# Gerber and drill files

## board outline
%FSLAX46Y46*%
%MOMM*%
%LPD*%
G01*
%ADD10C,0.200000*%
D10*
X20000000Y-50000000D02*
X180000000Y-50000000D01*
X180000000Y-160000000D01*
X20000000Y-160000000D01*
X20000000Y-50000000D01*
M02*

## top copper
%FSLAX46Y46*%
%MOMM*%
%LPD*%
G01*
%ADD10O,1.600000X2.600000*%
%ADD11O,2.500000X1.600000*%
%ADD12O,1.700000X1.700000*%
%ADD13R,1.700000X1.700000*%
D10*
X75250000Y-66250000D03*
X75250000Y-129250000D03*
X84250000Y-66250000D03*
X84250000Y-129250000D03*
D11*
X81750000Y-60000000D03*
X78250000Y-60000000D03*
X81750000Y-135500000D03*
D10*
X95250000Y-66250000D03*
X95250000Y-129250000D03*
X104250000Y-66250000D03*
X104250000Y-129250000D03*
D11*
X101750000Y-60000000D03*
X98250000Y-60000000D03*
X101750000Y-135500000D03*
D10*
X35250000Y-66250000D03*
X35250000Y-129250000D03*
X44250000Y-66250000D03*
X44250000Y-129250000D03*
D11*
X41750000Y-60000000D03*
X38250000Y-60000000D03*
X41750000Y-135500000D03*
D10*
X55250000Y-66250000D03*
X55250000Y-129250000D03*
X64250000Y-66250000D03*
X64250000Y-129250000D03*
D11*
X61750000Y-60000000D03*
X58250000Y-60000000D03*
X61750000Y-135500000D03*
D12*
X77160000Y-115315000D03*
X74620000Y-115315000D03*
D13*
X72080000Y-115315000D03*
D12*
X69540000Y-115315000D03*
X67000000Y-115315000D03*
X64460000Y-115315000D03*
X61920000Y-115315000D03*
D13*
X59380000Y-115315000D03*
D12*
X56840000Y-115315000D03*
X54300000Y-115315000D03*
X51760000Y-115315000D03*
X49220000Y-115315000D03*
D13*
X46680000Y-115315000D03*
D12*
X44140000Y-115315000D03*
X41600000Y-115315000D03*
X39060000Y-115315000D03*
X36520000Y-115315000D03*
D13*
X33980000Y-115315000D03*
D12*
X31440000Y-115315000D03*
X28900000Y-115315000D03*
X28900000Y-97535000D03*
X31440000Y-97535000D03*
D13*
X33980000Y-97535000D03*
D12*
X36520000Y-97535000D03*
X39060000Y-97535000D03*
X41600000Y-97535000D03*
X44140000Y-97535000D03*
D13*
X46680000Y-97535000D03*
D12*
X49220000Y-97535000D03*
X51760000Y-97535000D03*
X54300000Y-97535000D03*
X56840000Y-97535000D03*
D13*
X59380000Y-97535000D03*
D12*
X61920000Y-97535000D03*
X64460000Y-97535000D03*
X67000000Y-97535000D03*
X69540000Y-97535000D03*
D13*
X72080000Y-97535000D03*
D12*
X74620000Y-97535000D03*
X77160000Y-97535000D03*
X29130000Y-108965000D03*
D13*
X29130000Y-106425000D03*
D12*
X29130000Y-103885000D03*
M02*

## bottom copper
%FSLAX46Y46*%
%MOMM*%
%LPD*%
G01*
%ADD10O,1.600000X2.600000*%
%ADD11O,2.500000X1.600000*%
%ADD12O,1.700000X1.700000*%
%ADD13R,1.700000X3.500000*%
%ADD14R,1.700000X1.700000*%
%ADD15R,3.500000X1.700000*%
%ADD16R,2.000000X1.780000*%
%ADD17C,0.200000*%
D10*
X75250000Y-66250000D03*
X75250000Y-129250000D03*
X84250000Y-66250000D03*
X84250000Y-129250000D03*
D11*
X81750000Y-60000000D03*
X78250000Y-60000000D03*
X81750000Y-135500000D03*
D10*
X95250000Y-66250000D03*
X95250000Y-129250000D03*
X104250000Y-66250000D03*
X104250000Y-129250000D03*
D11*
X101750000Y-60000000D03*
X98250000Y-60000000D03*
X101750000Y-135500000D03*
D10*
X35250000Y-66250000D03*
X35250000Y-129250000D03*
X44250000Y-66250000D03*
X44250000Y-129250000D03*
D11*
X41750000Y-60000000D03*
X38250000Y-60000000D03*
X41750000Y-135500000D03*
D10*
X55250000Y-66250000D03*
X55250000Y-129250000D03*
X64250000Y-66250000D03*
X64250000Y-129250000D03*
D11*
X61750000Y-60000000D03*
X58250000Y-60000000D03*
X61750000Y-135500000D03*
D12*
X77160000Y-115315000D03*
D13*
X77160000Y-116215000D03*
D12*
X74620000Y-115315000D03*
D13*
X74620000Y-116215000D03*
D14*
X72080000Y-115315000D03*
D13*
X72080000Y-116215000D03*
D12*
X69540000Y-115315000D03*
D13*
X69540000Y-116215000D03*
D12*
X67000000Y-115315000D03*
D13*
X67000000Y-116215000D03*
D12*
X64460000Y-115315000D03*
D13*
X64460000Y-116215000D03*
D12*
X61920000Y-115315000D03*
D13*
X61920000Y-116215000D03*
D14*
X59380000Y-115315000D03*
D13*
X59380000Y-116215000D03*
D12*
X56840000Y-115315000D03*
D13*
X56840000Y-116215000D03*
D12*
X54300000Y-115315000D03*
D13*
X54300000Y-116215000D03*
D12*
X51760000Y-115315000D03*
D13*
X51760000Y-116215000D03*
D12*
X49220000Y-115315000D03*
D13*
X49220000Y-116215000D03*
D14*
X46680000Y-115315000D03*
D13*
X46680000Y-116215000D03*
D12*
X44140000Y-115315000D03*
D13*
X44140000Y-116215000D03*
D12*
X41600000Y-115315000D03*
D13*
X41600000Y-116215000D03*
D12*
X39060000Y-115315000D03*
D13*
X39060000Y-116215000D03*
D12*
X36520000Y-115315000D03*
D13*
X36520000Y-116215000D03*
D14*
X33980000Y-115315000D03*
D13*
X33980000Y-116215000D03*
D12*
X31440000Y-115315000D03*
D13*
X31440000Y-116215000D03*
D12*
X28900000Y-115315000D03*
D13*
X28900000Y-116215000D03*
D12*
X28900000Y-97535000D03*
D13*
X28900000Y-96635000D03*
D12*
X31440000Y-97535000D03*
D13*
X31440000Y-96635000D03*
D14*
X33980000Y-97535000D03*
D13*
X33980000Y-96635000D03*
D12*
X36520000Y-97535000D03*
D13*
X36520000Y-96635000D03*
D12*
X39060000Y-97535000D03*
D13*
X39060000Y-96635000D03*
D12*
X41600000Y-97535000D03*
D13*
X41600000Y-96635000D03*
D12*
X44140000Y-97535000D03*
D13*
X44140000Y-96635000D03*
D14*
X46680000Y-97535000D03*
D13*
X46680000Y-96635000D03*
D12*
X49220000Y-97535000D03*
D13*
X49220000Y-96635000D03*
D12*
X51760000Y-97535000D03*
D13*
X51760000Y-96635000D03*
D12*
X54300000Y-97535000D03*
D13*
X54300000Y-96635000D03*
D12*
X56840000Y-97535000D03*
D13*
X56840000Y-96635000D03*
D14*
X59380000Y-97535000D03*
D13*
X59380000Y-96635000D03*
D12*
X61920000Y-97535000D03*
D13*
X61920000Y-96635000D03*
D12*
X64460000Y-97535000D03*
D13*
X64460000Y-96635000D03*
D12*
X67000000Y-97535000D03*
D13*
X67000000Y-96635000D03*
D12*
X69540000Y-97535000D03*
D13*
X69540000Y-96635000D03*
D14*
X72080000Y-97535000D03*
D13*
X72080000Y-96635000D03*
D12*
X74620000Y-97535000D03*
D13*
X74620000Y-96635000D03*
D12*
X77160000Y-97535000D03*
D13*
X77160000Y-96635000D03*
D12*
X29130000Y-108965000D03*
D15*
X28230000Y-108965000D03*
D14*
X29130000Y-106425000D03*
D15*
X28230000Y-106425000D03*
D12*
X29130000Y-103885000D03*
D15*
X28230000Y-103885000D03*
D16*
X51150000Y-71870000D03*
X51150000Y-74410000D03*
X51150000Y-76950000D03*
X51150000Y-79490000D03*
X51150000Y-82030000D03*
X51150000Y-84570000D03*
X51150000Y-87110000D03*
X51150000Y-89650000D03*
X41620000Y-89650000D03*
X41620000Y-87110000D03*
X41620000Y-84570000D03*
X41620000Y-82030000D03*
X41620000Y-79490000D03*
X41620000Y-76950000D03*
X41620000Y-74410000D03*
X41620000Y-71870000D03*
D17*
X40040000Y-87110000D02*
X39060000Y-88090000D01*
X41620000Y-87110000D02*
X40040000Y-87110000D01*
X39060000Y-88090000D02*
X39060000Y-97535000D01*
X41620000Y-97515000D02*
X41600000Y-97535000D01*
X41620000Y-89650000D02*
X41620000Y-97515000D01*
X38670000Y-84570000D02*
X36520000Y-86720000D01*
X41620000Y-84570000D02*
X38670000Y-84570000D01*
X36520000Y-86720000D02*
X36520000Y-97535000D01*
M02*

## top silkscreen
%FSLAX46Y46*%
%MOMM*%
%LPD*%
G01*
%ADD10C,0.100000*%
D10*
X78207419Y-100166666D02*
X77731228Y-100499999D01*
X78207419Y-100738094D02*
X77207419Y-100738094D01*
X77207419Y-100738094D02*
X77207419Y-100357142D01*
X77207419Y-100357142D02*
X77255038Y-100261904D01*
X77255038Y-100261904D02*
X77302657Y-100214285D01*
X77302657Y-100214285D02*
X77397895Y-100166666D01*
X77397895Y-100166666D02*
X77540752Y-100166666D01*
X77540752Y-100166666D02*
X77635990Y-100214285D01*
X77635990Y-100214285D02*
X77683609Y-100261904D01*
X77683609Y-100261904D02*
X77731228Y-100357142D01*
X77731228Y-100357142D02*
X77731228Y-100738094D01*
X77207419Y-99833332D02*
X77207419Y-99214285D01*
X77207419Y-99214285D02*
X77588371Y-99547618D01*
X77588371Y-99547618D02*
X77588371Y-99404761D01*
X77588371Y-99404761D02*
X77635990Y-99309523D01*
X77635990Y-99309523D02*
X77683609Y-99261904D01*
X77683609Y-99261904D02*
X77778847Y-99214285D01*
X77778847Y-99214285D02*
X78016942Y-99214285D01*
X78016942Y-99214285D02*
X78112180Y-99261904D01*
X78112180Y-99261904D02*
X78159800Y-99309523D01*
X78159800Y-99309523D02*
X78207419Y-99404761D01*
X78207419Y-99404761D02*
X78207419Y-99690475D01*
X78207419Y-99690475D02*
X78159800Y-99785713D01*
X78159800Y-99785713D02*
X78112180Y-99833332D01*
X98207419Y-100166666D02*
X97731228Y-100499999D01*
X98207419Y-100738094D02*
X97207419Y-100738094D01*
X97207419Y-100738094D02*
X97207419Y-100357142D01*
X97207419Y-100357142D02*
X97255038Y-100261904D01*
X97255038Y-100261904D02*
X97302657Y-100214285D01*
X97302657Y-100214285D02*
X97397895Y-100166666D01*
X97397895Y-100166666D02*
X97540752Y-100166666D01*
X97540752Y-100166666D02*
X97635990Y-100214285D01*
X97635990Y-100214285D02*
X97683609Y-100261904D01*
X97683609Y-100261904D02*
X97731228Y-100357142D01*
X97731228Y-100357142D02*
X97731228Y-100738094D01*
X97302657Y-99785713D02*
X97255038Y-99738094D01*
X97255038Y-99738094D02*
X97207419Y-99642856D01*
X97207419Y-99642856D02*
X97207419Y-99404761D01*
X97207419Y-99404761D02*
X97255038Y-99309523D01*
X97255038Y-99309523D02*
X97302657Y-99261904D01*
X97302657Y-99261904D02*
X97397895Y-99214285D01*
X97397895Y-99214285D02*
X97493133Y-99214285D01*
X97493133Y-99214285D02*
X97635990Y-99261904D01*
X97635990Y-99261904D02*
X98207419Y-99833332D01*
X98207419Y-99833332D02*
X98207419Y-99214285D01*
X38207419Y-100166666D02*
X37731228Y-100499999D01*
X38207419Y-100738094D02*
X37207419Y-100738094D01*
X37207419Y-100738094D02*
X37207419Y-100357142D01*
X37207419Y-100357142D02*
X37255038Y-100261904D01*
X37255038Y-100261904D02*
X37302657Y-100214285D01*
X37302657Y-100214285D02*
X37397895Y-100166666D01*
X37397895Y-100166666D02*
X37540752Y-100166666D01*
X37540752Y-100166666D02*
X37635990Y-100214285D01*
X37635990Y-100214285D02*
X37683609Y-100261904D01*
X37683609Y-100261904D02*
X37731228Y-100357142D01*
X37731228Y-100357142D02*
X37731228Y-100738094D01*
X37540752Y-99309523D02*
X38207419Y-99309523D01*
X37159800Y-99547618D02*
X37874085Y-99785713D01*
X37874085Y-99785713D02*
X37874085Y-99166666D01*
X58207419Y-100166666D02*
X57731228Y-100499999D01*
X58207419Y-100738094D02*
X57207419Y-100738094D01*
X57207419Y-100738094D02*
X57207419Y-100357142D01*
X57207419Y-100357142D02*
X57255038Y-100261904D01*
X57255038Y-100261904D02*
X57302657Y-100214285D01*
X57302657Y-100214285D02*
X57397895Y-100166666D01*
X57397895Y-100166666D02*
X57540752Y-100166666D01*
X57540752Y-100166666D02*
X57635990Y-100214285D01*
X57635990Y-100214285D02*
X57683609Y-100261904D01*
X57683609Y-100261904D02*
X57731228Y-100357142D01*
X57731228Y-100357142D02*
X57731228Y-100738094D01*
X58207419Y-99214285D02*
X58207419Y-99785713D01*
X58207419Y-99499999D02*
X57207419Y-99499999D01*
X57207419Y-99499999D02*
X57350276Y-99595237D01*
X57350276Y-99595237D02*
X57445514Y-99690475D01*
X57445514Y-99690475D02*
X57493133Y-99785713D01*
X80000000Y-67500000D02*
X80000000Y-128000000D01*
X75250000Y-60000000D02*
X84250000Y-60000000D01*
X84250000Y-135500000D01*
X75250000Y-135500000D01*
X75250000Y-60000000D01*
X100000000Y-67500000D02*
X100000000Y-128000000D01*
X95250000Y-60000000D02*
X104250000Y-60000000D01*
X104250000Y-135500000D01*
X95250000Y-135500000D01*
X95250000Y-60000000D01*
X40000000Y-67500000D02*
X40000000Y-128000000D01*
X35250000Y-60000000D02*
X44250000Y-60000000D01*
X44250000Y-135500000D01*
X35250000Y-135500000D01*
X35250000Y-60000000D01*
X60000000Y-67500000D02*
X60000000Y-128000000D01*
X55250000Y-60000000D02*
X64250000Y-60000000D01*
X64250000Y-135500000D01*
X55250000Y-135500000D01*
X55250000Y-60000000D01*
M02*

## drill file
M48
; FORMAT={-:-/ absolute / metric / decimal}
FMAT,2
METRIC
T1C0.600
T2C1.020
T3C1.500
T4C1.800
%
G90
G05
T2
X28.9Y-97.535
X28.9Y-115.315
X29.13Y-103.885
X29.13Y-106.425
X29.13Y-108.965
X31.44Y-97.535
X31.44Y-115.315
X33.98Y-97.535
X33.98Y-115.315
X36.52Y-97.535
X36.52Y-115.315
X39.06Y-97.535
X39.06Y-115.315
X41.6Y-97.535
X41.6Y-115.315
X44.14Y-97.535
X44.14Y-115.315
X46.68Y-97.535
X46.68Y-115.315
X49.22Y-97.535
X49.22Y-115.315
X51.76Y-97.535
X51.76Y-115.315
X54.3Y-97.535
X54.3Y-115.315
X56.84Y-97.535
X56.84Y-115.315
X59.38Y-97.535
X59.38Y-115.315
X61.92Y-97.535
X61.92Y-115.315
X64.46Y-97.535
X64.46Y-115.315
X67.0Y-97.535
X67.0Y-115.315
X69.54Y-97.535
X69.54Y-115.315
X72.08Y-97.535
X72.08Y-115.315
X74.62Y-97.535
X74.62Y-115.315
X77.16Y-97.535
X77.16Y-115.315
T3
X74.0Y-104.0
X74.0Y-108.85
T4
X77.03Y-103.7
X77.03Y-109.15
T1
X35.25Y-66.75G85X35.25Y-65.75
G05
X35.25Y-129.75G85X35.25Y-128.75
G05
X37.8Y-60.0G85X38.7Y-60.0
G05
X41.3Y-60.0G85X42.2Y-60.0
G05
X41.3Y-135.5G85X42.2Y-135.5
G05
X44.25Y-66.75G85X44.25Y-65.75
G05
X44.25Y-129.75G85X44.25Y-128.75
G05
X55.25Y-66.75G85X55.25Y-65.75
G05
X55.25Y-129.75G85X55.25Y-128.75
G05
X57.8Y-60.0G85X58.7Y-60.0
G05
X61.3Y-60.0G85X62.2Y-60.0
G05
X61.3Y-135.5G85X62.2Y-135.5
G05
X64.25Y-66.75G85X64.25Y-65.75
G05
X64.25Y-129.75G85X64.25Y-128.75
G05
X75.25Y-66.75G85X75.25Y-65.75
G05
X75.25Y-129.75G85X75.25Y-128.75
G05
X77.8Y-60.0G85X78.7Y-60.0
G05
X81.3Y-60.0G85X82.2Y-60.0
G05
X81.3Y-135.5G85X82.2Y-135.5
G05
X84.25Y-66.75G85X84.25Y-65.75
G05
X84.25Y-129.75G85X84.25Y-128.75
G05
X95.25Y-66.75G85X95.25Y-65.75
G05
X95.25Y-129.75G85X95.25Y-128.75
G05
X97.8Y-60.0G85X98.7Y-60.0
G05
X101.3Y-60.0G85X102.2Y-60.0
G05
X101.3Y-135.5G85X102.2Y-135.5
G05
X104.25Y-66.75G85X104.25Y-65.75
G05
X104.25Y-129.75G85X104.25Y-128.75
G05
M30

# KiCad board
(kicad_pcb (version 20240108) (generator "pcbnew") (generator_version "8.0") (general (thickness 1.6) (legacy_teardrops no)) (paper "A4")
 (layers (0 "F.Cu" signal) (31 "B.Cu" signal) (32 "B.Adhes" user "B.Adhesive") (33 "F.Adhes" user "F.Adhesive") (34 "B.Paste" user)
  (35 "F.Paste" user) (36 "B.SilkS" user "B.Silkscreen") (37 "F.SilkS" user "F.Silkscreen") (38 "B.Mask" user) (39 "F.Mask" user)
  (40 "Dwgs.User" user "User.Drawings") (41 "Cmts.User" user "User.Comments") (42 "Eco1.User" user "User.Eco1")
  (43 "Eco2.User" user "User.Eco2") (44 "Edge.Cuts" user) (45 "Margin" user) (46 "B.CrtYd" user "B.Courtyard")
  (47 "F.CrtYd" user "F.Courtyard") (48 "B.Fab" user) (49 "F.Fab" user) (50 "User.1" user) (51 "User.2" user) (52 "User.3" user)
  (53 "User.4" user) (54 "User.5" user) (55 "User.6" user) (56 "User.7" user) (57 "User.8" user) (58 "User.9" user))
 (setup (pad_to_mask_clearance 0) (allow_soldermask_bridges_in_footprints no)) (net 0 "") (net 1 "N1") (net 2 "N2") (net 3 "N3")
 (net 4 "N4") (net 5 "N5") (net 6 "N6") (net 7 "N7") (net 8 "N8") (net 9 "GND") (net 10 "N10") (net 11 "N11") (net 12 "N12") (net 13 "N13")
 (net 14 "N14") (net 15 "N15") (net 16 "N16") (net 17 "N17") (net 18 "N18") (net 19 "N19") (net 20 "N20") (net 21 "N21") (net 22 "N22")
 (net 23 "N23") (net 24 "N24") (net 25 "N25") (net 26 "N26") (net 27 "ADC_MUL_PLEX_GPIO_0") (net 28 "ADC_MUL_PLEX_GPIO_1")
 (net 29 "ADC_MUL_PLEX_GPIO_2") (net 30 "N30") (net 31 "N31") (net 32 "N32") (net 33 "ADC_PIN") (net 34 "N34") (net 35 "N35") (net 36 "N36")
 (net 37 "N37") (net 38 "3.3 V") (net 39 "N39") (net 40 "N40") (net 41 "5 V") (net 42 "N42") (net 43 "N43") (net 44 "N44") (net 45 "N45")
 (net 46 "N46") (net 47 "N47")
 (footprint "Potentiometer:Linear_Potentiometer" (layer "F.Cu") (at 80 60)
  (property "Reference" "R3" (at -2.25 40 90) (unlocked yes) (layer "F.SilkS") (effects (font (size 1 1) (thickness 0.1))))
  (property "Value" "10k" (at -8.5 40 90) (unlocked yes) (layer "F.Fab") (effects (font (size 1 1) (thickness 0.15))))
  (fp_line (start 0 7.5) (end 0 68) (stroke (width 0.1) (type default)) (layer "F.SilkS"))
  (fp_rect (start -4.75 0) (end 4.25 75.5) (stroke (width 0.1) (type default)) (fill none) (layer "F.SilkS"))
  (pad "0" thru_hole oval (at -4.75 6.25 180) (size 1.6 2.6) (drill oval 0.6 1.6) (layers "*.Cu" "*.Mask") (remove_unused_layers no))
  (pad "0" thru_hole oval (at -4.75 69.25 180) (size 1.6 2.6) (drill oval 0.6 1.6) (layers "*.Cu" "*.Mask") (remove_unused_layers no))
  (pad "0" thru_hole oval (at 4.25 6.25 180) (size 1.6 2.6) (drill oval 0.6 1.6) (layers "*.Cu" "*.Mask") (remove_unused_layers no))
  (pad "0" thru_hole oval (at 4.25 69.25 180) (size 1.6 2.6) (drill oval 0.6 1.6) (layers "*.Cu" "*.Mask") (remove_unused_layers no))
  (pad "1" thru_hole oval (at 1.75 0) (size 2.5 1.6) (drill oval 1.5 0.6) (layers "*.Cu" "*.Mask") (remove_unused_layers no) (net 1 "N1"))
  (pad "2" thru_hole oval (at -1.75 0) (size 2.5 1.6) (drill oval 1.5 0.6) (layers "*.Cu" "*.Mask") (remove_unused_layers no) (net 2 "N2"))
  (pad "3" thru_hole oval (at 1.75 75.5) (size 2.5 1.6) (drill oval 1.5 0.6) (layers "*.Cu" "*.Mask") (remove_unused_layers no) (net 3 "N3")))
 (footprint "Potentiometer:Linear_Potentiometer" (layer "F.Cu") (at 100 60)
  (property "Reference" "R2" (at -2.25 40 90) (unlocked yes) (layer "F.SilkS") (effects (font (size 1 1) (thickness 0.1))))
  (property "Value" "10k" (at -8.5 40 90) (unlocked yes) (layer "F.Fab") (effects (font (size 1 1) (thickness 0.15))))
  (fp_line (start 0 7.5) (end 0 68) (stroke (width 0.1) (type default)) (layer "F.SilkS"))
  (fp_rect (start -4.75 0) (end 4.25 75.5) (stroke (width 0.1) (type default)) (fill none) (layer "F.SilkS"))
  (pad "0" thru_hole oval (at -4.75 6.25 180) (size 1.6 2.6) (drill oval 0.6 1.6) (layers "*.Cu" "*.Mask") (remove_unused_layers no))
  (pad "0" thru_hole oval (at -4.75 69.25 180) (size 1.6 2.6) (drill oval 0.6 1.6) (layers "*.Cu" "*.Mask") (remove_unused_layers no))
  (pad "0" thru_hole oval (at 4.25 6.25 180) (size 1.6 2.6) (drill oval 0.6 1.6) (layers "*.Cu" "*.Mask") (remove_unused_layers no))
  (pad "0" thru_hole oval (at 4.25 69.25 180) (size 1.6 2.6) (drill oval 0.6 1.6) (layers "*.Cu" "*.Mask") (remove_unused_layers no))
  (pad "1" thru_hole oval (at 1.75 0) (size 2.5 1.6) (drill oval 1.5 0.6) (layers "*.Cu" "*.Mask") (remove_unused_layers no) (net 1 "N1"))
  (pad "2" thru_hole oval (at -1.75 0) (size 2.5 1.6) (drill oval 1.5 0.6) (layers "*.Cu" "*.Mask") (remove_unused_layers no) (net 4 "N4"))
  (pad "3" thru_hole oval (at 1.75 75.5) (size 2.5 1.6) (drill oval 1.5 0.6) (layers "*.Cu" "*.Mask") (remove_unused_layers no) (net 3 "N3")))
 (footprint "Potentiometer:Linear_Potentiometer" (layer "F.Cu") (at 40 60)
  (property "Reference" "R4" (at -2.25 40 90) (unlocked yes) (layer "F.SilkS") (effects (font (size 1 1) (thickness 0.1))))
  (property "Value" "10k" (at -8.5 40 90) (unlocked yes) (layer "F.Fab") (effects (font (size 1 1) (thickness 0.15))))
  (fp_line (start 0 7.5) (end 0 68) (stroke (width 0.1) (type default)) (layer "F.SilkS"))
  (fp_rect (start -4.75 0) (end 4.25 75.5) (stroke (width 0.1) (type default)) (fill none) (layer "F.SilkS"))
  (pad "0" thru_hole oval (at -4.75 6.25 180) (size 1.6 2.6) (drill oval 0.6 1.6) (layers "*.Cu" "*.Mask") (remove_unused_layers no))
  (pad "0" thru_hole oval (at -4.75 69.25 180) (size 1.6 2.6) (drill oval 0.6 1.6) (layers "*.Cu" "*.Mask") (remove_unused_layers no))
  (pad "0" thru_hole oval (at 4.25 6.25 180) (size 1.6 2.6) (drill oval 0.6 1.6) (layers "*.Cu" "*.Mask") (remove_unused_layers no))
  (pad "0" thru_hole oval (at 4.25 69.25 180) (size 1.6 2.6) (drill oval 0.6 1.6) (layers "*.Cu" "*.Mask") (remove_unused_layers no))
  (pad "1" thru_hole oval (at 1.75 0) (size 2.5 1.6) (drill oval 1.5 0.6) (layers "*.Cu" "*.Mask") (remove_unused_layers no) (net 1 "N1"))
  (pad "2" thru_hole oval (at -1.75 0) (size 2.5 1.6) (drill oval 1.5 0.6) (layers "*.Cu" "*.Mask") (remove_unused_layers no) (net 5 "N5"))
  (pad "3" thru_hole oval (at 1.75 75.5) (size 2.5 1.6) (drill oval 1.5 0.6) (layers "*.Cu" "*.Mask") (remove_unused_layers no) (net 3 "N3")))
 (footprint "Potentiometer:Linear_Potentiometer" (layer "F.Cu") (at 60 60)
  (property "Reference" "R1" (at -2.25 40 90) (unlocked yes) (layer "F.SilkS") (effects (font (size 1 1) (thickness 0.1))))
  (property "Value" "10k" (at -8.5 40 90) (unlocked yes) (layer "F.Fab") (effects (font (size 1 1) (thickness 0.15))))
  (fp_line (start 0 7.5) (end 0 68) (stroke (width 0.1) (type default)) (layer "F.SilkS"))
  (fp_rect (start -4.75 0) (end 4.25 75.5) (stroke (width 0.1) (type default)) (fill none) (layer "F.SilkS"))
  (pad "0" thru_hole oval (at -4.75 6.25 180) (size 1.6 2.6) (drill oval 0.6 1.6) (layers "*.Cu" "*.Mask") (remove_unused_layers no))
  (pad "0" thru_hole oval (at -4.75 69.25 180) (size 1.6 2.6) (drill oval 0.6 1.6) (layers "*.Cu" "*.Mask") (remove_unused_layers no))
  (pad "0" thru_hole oval (at 4.25 6.25 180) (size 1.6 2.6) (drill oval 0.6 1.6) (layers "*.Cu" "*.Mask") (remove_unused_layers no))
  (pad "0" thru_hole oval (at 4.25 69.25 180) (size 1.6 2.6) (drill oval 0.6 1.6) (layers "*.Cu" "*.Mask") (remove_unused_layers no))
  (pad "1" thru_hole oval (at 1.75 0) (size 2.5 1.6) (drill oval 1.5 0.6) (layers "*.Cu" "*.Mask") (remove_unused_layers no) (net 1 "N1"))
  (pad "2" thru_hole oval (at -1.75 0) (size 2.5 1.6) (drill oval 1.5 0.6) (layers "*.Cu" "*.Mask") (remove_unused_layers no) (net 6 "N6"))
  (pad "3" thru_hole oval (at 1.75 75.5) (size 2.5 1.6) (drill oval 1.5 0.6) (layers "*.Cu" "*.Mask") (remove_unused_layers no) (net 3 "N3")))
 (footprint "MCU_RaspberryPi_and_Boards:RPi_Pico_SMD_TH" (layer "B.Cu") (at 53.03 106.425 90)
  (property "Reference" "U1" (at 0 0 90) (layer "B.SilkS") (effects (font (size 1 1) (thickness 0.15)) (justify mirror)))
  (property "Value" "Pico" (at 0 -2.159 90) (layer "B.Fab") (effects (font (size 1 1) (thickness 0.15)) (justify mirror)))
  (pad "" np_thru_hole oval (at -2.725 24 90) (size 1.8 1.8) (drill 1.8) (layers "*.Cu" "*.Mask"))
  (pad "" np_thru_hole oval (at -2.425 20.97 90) (size 1.5 1.5) (drill 1.5) (layers "*.Cu" "*.Mask"))
  (pad "" np_thru_hole oval (at 2.425 20.97 90) (size 1.5 1.5) (drill 1.5) (layers "*.Cu" "*.Mask"))
  (pad "" np_thru_hole oval (at 2.725 24 90) (size 1.8 1.8) (drill 1.8) (layers "*.Cu" "*.Mask"))
  (pad "1" thru_hole oval (at -8.89 24.13 90) (size 1.7 1.7) (drill 1.02) (layers "*.Cu" "*.Mask") (remove_unused_layers no) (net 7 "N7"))
  (pad "1" smd rect (at -8.89 24.13 90) (size 3.5 1.7) (drill (offset -0.9 0)) (layers "B.Cu" "B.Mask") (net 7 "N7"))
  (pad "2" thru_hole oval (at -8.89 21.59 90) (size 1.7 1.7) (drill 1.02) (layers "*.Cu" "*.Mask") (remove_unused_layers no) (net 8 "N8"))
  (pad "2" smd rect (at -8.89 21.59 90) (size 3.5 1.7) (drill (offset -0.9 0)) (layers "B.Cu" "B.Mask") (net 8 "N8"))
  (pad "3" thru_hole rect (at -8.89 19.05 90) (size 1.7 1.7) (drill 1.02) (layers "*.Cu" "*.Mask") (remove_unused_layers no) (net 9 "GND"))
  (pad "3" smd rect (at -8.89 19.05 90) (size 3.5 1.7) (drill (offset -0.9 0)) (layers "B.Cu" "B.Mask") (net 9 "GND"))
  (pad "4" thru_hole oval (at -8.89 16.51 90) (size 1.7 1.7) (drill 1.02) (layers "*.Cu" "*.Mask") (remove_unused_layers no) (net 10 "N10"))
  (pad "4" smd rect (at -8.89 16.51 90) (size 3.5 1.7) (drill (offset -0.9 0)) (layers "B.Cu" "B.Mask") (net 10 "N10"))
  (pad "5" thru_hole oval (at -8.89 13.97 90) (size 1.7 1.7) (drill 1.02) (layers "*.Cu" "*.Mask") (remove_unused_layers no) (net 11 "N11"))
  (pad "5" smd rect (at -8.89 13.97 90) (size 3.5 1.7) (drill (offset -0.9 0)) (layers "B.Cu" "B.Mask") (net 11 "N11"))
  (pad "6" thru_hole oval (at -8.89 11.43 90) (size 1.7 1.7) (drill 1.02) (layers "*.Cu" "*.Mask") (remove_unused_layers no) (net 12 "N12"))
  (pad "6" smd rect (at -8.89 11.43 90) (size 3.5 1.7) (drill (offset -0.9 0)) (layers "B.Cu" "B.Mask") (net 12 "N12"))
  (pad "7" thru_hole oval (at -8.89 8.89 90) (size 1.7 1.7) (drill 1.02) (layers "*.Cu" "*.Mask") (remove_unused_layers no) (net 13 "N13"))
  (pad "7" smd rect (at -8.89 8.89 90) (size 3.5 1.7) (drill (offset -0.9 0)) (layers "B.Cu" "B.Mask") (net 13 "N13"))
  (pad "8" thru_hole rect (at -8.89 6.35 90) (size 1.7 1.7) (drill 1.02) (layers "*.Cu" "*.Mask") (remove_unused_layers no) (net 9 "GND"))
  (pad "8" smd rect (at -8.89 6.35 90) (size 3.5 1.7) (drill (offset -0.9 0)) (layers "B.Cu" "B.Mask") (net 9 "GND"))
  (pad "9" thru_hole oval (at -8.89 3.81 90) (size 1.7 1.7) (drill 1.02) (layers "*.Cu" "*.Mask") (remove_unused_layers no) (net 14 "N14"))
  (pad "9" smd rect (at -8.89 3.81 90) (size 3.5 1.7) (drill (offset -0.9 0)) (layers "B.Cu" "B.Mask") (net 14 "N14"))
  (pad "10" thru_hole oval (at -8.89 1.27 90) (size 1.7 1.7) (drill 1.02) (layers "*.Cu" "*.Mask") (remove_unused_layers no) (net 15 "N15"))
  (pad "10" smd rect (at -8.89 1.27 90) (size 3.5 1.7) (drill (offset -0.9 0)) (layers "B.Cu" "B.Mask") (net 15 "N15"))
  (pad "11" thru_hole oval (at -8.89 -1.27 90) (size 1.7 1.7) (drill 1.02) (layers "*.Cu" "*.Mask") (remove_unused_layers no) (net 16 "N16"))
  (pad "11" smd rect (at -8.89 -1.27 90) (size 3.5 1.7) (drill (offset -0.9 0)) (layers "B.Cu" "B.Mask") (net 16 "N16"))
  (pad "12" thru_hole oval (at -8.89 -3.81 90) (size 1.7 1.7) (drill 1.02) (layers "*.Cu" "*.Mask") (remove_unused_layers no) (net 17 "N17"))
  (pad "12" smd rect (at -8.89 -3.81 90) (size 3.5 1.7) (drill (offset -0.9 0)) (layers "B.Cu" "B.Mask") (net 17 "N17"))
  (pad "13" thru_hole rect (at -8.89 -6.35 90) (size 1.7 1.7) (drill 1.02) (layers "*.Cu" "*.Mask") (remove_unused_layers no) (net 9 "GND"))
  (pad "13" smd rect (at -8.89 -6.35 90) (size 3.5 1.7) (drill (offset -0.9 0)) (layers "B.Cu" "B.Mask") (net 9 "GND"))
  (pad "14" thru_hole oval (at -8.89 -8.89 90) (size 1.7 1.7) (drill 1.02) (layers "*.Cu" "*.Mask") (remove_unused_layers no) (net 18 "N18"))
  (pad "14" smd rect (at -8.89 -8.89 90) (size 3.5 1.7) (drill (offset -0.9 0)) (layers "B.Cu" "B.Mask") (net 18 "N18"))
  (pad "15" thru_hole oval (at -8.89 -11.43 90) (size 1.7 1.7) (drill 1.02) (layers "*.Cu" "*.Mask") (remove_unused_layers no)
   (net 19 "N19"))
  (pad "15" smd rect (at -8.89 -11.43 90) (size 3.5 1.7) (drill (offset -0.9 0)) (layers "B.Cu" "B.Mask") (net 19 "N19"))
  (pad "16" thru_hole oval (at -8.89 -13.97 90) (size 1.7 1.7) (drill 1.02) (layers "*.Cu" "*.Mask") (remove_unused_layers no)
   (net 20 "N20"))
  (pad "16" smd rect (at -8.89 -13.97 90) (size 3.5 1.7) (drill (offset -0.9 0)) (layers "B.Cu" "B.Mask") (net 20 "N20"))
  (pad "17" thru_hole oval (at -8.89 -16.51 90) (size 1.7 1.7) (drill 1.02) (layers "*.Cu" "*.Mask") (remove_unused_layers no)
   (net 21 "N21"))
  (pad "17" smd rect (at -8.89 -16.51 90) (size 3.5 1.7) (drill (offset -0.9 0)) (layers "B.Cu" "B.Mask") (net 21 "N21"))
  (pad "18" thru_hole rect (at -8.89 -19.05 90) (size 1.7 1.7) (drill 1.02) (layers "*.Cu" "*.Mask") (remove_unused_layers no)
   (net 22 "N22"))
  (pad "18" smd rect (at -8.89 -19.05 90) (size 3.5 1.7) (drill (offset -0.9 0)) (layers "B.Cu" "B.Mask") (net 22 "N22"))
  (pad "19" thru_hole oval (at -8.89 -21.59 90) (size 1.7 1.7) (drill 1.02) (layers "*.Cu" "*.Mask") (remove_unused_layers no)
   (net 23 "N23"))
  (pad "19" smd rect (at -8.89 -21.59 90) (size 3.5 1.7) (drill (offset -0.9 0)) (layers "B.Cu" "B.Mask") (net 23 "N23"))
  (pad "20" thru_hole oval (at -8.89 -24.13 90) (size 1.7 1.7) (drill 1.02) (layers "*.Cu" "*.Mask") (remove_unused_layers no)
   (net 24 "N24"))
  (pad "20" smd rect (at -8.89 -24.13 90) (size 3.5 1.7) (drill (offset -0.9 0)) (layers "B.Cu" "B.Mask") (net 24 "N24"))
  (pad "21" thru_hole oval (at 8.89 -24.13 90) (size 1.7 1.7) (drill 1.02) (layers "*.Cu" "*.Mask") (remove_unused_layers no) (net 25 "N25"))
  (pad "21" smd rect (at 8.89 -24.13 90) (size 3.5 1.7) (drill (offset 0.9 0)) (layers "B.Cu" "B.Mask") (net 25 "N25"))
  (pad "22" thru_hole oval (at 8.89 -21.59 90) (size 1.7 1.7) (drill 1.02) (layers "*.Cu" "*.Mask") (remove_unused_layers no) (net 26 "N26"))
  (pad "22" smd rect (at 8.89 -21.59 90) (size 3.5 1.7) (drill (offset 0.9 0)) (layers "B.Cu" "B.Mask") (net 26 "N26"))
  (pad "23" thru_hole rect (at 8.89 -19.05 90) (size 1.7 1.7) (drill 1.02) (layers "*.Cu" "*.Mask") (remove_unused_layers no) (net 9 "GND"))
  (pad "23" smd rect (at 8.89 -19.05 90) (size 3.5 1.7) (drill (offset 0.9 0)) (layers "B.Cu" "B.Mask") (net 9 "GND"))
  (pad "24" thru_hole oval (at 8.89 -16.51 90) (size 1.7 1.7) (drill 1.02) (layers "*.Cu" "*.Mask") (remove_unused_layers no)
   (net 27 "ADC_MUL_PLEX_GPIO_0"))
  (pad "24" smd rect (at 8.89 -16.51 90) (size 3.5 1.7) (drill (offset 0.9 0)) (layers "B.Cu" "B.Mask") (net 27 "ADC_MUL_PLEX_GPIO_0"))
  (pad "25" thru_hole oval (at 8.89 -13.97 90) (size 1.7 1.7) (drill 1.02) (layers "*.Cu" "*.Mask") (remove_unused_layers no)
   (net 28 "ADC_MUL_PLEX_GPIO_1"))
  (pad "25" smd rect (at 8.89 -13.97 90) (size 3.5 1.7) (drill (offset 0.9 0)) (layers "B.Cu" "B.Mask") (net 28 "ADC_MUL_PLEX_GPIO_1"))
  (pad "26" thru_hole oval (at 8.89 -11.43 90) (size 1.7 1.7) (drill 1.02) (layers "*.Cu" "*.Mask") (remove_unused_layers no)
   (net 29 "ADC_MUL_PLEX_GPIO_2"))
  (pad "26" smd rect (at 8.89 -11.43 90) (size 3.5 1.7) (drill (offset 0.9 0)) (layers "B.Cu" "B.Mask") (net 29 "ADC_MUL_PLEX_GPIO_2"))
  (pad "27" thru_hole oval (at 8.89 -8.89 90) (size 1.7 1.7) (drill 1.02) (layers "*.Cu" "*.Mask") (remove_unused_layers no) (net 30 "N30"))
  (pad "27" smd rect (at 8.89 -8.89 90) (size 3.5 1.7) (drill (offset 0.9 0)) (layers "B.Cu" "B.Mask") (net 30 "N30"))
  (pad "28" thru_hole rect (at 8.89 -6.35 90) (size 1.7 1.7) (drill 1.02) (layers "*.Cu" "*.Mask") (remove_unused_layers no) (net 9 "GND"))
  (pad "28" smd rect (at 8.89 -6.35 90) (size 3.5 1.7) (drill (offset 0.9 0)) (layers "B.Cu" "B.Mask") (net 9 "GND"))
  (pad "29" thru_hole oval (at 8.89 -3.81 90) (size 1.7 1.7) (drill 1.02) (layers "*.Cu" "*.Mask") (remove_unused_layers no) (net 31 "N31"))
  (pad "29" smd rect (at 8.89 -3.81 90) (size 3.5 1.7) (drill (offset 0.9 0)) (layers "B.Cu" "B.Mask") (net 31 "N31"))
  (pad "30" thru_hole oval (at 8.89 -1.27 90) (size 1.7 1.7) (drill 1.02) (layers "*.Cu" "*.Mask") (remove_unused_layers no) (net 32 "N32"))
  (pad "30" smd rect (at 8.89 -1.27 90) (size 3.5 1.7) (drill (offset 0.9 0)) (layers "B.Cu" "B.Mask") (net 32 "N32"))
  (pad "31" thru_hole oval (at 8.89 1.27 90) (size 1.7 1.7) (drill 1.02) (layers "*.Cu" "*.Mask") (remove_unused_layers no)
   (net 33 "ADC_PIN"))
  (pad "31" smd rect (at 8.89 1.27 90) (size 3.5 1.7) (drill (offset 0.9 0)) (layers "B.Cu" "B.Mask") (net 33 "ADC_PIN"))
  (pad "32" thru_hole oval (at 8.89 3.81 90) (size 1.7 1.7) (drill 1.02) (layers "*.Cu" "*.Mask") (remove_unused_layers no) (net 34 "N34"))
  (pad "32" smd rect (at 8.89 3.81 90) (size 3.5 1.7) (drill (offset 0.9 0)) (layers "B.Cu" "B.Mask") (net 34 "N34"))
  (pad "33" thru_hole rect (at 8.89 6.35 90) (size 1.7 1.7) (drill 1.02) (layers "*.Cu" "*.Mask") (remove_unused_layers no) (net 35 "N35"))
  (pad "33" smd rect (at 8.89 6.35 90) (size 3.5 1.7) (drill (offset 0.9 0)) (layers "B.Cu" "B.Mask") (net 35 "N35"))
  (pad "34" thru_hole oval (at 8.89 8.89 90) (size 1.7 1.7) (drill 1.02) (layers "*.Cu" "*.Mask") (remove_unused_layers no) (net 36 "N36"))
  (pad "34" smd rect (at 8.89 8.89 90) (size 3.5 1.7) (drill (offset 0.9 0)) (layers "B.Cu" "B.Mask") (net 36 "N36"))
  (pad "35" thru_hole oval (at 8.89 11.43 90) (size 1.7 1.7) (drill 1.02) (layers "*.Cu" "*.Mask") (remove_unused_layers no) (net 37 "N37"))
  (pad "35" smd rect (at 8.89 11.43 90) (size 3.5 1.7) (drill (offset 0.9 0)) (layers "B.Cu" "B.Mask") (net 37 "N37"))
  (pad "36" thru_hole oval (at 8.89 13.97 90) (size 1.7 1.7) (drill 1.02) (layers "*.Cu" "*.Mask") (remove_unused_layers no)
   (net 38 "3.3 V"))
  (pad "36" smd rect (at 8.89 13.97 90) (size 3.5 1.7) (drill (offset 0.9 0)) (layers "B.Cu" "B.Mask") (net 38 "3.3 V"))
  (pad "37" thru_hole oval (at 8.89 16.51 90) (size 1.7 1.7) (drill 1.02) (layers "*.Cu" "*.Mask") (remove_unused_layers no) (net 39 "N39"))
  (pad "37" smd rect (at 8.89 16.51 90) (size 3.5 1.7) (drill (offset 0.9 0)) (layers "B.Cu" "B.Mask") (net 39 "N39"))
  (pad "38" thru_hole rect (at 8.89 19.05 90) (size 1.7 1.7) (drill 1.02) (layers "*.Cu" "*.Mask") (remove_unused_layers no) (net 9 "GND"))
  (pad "38" smd rect (at 8.89 19.05 90) (size 3.5 1.7) (drill (offset 0.9 0)) (layers "B.Cu" "B.Mask") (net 9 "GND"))
  (pad "39" thru_hole oval (at 8.89 21.59 90) (size 1.7 1.7) (drill 1.02) (layers "*.Cu" "*.Mask") (remove_unused_layers no) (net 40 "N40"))
  (pad "39" smd rect (at 8.89 21.59 90) (size 3.5 1.7) (drill (offset 0.9 0)) (layers "B.Cu" "B.Mask") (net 40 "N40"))
  (pad "40" thru_hole oval (at 8.89 24.13 90) (size 1.7 1.7) (drill 1.02) (layers "*.Cu" "*.Mask") (remove_unused_layers no) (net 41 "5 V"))
  (pad "40" smd rect (at 8.89 24.13 90) (size 3.5 1.7) (drill (offset 0.9 0)) (layers "B.Cu" "B.Mask") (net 41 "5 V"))
  (pad "41" thru_hole oval (at -2.54 -23.9 90) (size 1.7 1.7) (drill 1.02) (layers "*.Cu" "*.Mask") (remove_unused_layers no) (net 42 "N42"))
  (pad "41" smd rect (at -2.54 -23.9) (size 3.5 1.7) (drill (offset -0.9 0)) (layers "B.Cu" "B.Mask") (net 42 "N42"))
  (pad "42" thru_hole rect (at 0 -23.9 90) (size 1.7 1.7) (drill 1.02) (layers "*.Cu" "*.Mask") (remove_unused_layers no) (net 9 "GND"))
  (pad "42" smd rect (at 0 -23.9) (size 3.5 1.7) (drill (offset -0.9 0)) (layers "B.Cu" "B.Mask") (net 9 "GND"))
  (pad "43" thru_hole oval (at 2.54 -23.9 90) (size 1.7 1.7) (drill 1.02) (layers "*.Cu" "*.Mask") (remove_unused_layers no) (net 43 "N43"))
  (pad "43" smd rect (at 2.54 -23.9) (size 3.5 1.7) (drill (offset -0.9 0)) (layers "B.Cu" "B.Mask") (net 43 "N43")))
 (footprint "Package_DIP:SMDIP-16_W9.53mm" (layer "B.Cu") (at 46.385 80.76 180)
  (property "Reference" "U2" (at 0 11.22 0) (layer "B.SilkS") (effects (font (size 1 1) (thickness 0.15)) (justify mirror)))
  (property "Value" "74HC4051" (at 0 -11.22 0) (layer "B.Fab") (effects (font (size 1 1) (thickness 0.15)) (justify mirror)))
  (pad "1" smd rect (at -4.765 8.89 180) (size 2 1.78) (layers "B.Cu" "B.Paste" "B.Mask") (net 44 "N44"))
  (pad "2" smd rect (at -4.765 6.35 180) (size 2 1.78) (layers "B.Cu" "B.Paste" "B.Mask") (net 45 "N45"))
  (pad "3" smd rect (at -4.765 3.81 180) (size 2 1.78) (layers "B.Cu" "B.Paste" "B.Mask") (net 33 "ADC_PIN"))
  (pad "4" smd rect (at -4.765 1.27 180) (size 2 1.78) (layers "B.Cu" "B.Paste" "B.Mask") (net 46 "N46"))
  (pad "5" smd rect (at -4.765 -1.27 180) (size 2 1.78) (layers "B.Cu" "B.Paste" "B.Mask") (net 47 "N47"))
  (pad "6" smd rect (at -4.765 -3.81 180) (size 2 1.78) (layers "B.Cu" "B.Paste" "B.Mask") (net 9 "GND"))
  (pad "7" smd rect (at -4.765 -6.35 180) (size 2 1.78) (layers "B.Cu" "B.Paste" "B.Mask") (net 9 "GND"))
  (pad "8" smd rect (at -4.765 -8.89 180) (size 2 1.78) (layers "B.Cu" "B.Paste" "B.Mask") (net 9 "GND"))
  (pad "9" smd rect (at 4.765 -8.89 180) (size 2 1.78) (layers "B.Cu" "B.Paste" "B.Mask") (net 29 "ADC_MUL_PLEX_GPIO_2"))
  (pad "10" smd rect (at 4.765 -6.35 180) (size 2 1.78) (layers "B.Cu" "B.Paste" "B.Mask") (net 28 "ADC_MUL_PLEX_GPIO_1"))
  (pad "11" smd rect (at 4.765 -3.81 180) (size 2 1.78) (layers "B.Cu" "B.Paste" "B.Mask") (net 27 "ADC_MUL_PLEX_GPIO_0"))
  (pad "12" smd rect (at 4.765 -1.27 180) (size 2 1.78) (layers "B.Cu" "B.Paste" "B.Mask") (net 5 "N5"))
  (pad "13" smd rect (at 4.765 1.27 180) (size 2 1.78) (layers "B.Cu" "B.Paste" "B.Mask") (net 6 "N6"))
  (pad "14" smd rect (at 4.765 3.81 180) (size 2 1.78) (layers "B.Cu" "B.Paste" "B.Mask") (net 4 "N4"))
  (pad "15" smd rect (at 4.765 6.35 180) (size 2 1.78) (layers "B.Cu" "B.Paste" "B.Mask") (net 2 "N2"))
  (pad "16" smd rect (at 4.765 8.89 180) (size 2 1.78) (layers "B.Cu" "B.Paste" "B.Mask") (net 38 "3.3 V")))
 (gr_rect (start 20 50) (end 180 160) (stroke (width 0.2) (type default)) (fill none) (layer "Edge.Cuts"))
 (segment (start 40.04 87.11) (end 39.06 88.09) (width 0.2) (layer "B.Cu") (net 28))
 (segment (start 41.62 87.11) (end 40.04 87.11) (width 0.2) (layer "B.Cu") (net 28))
 (segment (start 39.06 88.09) (end 39.06 97.535) (width 0.2) (layer "B.Cu") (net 28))
 (segment (start 41.62 97.515) (end 41.6 97.535) (width 0.2) (layer "B.Cu") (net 29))
 (segment (start 41.62 89.65) (end 41.62 97.515) (width 0.2) (layer "B.Cu") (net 29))
 (segment (start 38.67 84.57) (end 36.52 86.72) (width 0.2) (layer "B.Cu") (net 27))
 (segment (start 41.62 84.57) (end 38.67 84.57) (width 0.2) (layer "B.Cu") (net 27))
 (segment (start 36.52 86.72) (end 36.52 97.535) (width 0.2) (layer "B.Cu") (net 27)))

